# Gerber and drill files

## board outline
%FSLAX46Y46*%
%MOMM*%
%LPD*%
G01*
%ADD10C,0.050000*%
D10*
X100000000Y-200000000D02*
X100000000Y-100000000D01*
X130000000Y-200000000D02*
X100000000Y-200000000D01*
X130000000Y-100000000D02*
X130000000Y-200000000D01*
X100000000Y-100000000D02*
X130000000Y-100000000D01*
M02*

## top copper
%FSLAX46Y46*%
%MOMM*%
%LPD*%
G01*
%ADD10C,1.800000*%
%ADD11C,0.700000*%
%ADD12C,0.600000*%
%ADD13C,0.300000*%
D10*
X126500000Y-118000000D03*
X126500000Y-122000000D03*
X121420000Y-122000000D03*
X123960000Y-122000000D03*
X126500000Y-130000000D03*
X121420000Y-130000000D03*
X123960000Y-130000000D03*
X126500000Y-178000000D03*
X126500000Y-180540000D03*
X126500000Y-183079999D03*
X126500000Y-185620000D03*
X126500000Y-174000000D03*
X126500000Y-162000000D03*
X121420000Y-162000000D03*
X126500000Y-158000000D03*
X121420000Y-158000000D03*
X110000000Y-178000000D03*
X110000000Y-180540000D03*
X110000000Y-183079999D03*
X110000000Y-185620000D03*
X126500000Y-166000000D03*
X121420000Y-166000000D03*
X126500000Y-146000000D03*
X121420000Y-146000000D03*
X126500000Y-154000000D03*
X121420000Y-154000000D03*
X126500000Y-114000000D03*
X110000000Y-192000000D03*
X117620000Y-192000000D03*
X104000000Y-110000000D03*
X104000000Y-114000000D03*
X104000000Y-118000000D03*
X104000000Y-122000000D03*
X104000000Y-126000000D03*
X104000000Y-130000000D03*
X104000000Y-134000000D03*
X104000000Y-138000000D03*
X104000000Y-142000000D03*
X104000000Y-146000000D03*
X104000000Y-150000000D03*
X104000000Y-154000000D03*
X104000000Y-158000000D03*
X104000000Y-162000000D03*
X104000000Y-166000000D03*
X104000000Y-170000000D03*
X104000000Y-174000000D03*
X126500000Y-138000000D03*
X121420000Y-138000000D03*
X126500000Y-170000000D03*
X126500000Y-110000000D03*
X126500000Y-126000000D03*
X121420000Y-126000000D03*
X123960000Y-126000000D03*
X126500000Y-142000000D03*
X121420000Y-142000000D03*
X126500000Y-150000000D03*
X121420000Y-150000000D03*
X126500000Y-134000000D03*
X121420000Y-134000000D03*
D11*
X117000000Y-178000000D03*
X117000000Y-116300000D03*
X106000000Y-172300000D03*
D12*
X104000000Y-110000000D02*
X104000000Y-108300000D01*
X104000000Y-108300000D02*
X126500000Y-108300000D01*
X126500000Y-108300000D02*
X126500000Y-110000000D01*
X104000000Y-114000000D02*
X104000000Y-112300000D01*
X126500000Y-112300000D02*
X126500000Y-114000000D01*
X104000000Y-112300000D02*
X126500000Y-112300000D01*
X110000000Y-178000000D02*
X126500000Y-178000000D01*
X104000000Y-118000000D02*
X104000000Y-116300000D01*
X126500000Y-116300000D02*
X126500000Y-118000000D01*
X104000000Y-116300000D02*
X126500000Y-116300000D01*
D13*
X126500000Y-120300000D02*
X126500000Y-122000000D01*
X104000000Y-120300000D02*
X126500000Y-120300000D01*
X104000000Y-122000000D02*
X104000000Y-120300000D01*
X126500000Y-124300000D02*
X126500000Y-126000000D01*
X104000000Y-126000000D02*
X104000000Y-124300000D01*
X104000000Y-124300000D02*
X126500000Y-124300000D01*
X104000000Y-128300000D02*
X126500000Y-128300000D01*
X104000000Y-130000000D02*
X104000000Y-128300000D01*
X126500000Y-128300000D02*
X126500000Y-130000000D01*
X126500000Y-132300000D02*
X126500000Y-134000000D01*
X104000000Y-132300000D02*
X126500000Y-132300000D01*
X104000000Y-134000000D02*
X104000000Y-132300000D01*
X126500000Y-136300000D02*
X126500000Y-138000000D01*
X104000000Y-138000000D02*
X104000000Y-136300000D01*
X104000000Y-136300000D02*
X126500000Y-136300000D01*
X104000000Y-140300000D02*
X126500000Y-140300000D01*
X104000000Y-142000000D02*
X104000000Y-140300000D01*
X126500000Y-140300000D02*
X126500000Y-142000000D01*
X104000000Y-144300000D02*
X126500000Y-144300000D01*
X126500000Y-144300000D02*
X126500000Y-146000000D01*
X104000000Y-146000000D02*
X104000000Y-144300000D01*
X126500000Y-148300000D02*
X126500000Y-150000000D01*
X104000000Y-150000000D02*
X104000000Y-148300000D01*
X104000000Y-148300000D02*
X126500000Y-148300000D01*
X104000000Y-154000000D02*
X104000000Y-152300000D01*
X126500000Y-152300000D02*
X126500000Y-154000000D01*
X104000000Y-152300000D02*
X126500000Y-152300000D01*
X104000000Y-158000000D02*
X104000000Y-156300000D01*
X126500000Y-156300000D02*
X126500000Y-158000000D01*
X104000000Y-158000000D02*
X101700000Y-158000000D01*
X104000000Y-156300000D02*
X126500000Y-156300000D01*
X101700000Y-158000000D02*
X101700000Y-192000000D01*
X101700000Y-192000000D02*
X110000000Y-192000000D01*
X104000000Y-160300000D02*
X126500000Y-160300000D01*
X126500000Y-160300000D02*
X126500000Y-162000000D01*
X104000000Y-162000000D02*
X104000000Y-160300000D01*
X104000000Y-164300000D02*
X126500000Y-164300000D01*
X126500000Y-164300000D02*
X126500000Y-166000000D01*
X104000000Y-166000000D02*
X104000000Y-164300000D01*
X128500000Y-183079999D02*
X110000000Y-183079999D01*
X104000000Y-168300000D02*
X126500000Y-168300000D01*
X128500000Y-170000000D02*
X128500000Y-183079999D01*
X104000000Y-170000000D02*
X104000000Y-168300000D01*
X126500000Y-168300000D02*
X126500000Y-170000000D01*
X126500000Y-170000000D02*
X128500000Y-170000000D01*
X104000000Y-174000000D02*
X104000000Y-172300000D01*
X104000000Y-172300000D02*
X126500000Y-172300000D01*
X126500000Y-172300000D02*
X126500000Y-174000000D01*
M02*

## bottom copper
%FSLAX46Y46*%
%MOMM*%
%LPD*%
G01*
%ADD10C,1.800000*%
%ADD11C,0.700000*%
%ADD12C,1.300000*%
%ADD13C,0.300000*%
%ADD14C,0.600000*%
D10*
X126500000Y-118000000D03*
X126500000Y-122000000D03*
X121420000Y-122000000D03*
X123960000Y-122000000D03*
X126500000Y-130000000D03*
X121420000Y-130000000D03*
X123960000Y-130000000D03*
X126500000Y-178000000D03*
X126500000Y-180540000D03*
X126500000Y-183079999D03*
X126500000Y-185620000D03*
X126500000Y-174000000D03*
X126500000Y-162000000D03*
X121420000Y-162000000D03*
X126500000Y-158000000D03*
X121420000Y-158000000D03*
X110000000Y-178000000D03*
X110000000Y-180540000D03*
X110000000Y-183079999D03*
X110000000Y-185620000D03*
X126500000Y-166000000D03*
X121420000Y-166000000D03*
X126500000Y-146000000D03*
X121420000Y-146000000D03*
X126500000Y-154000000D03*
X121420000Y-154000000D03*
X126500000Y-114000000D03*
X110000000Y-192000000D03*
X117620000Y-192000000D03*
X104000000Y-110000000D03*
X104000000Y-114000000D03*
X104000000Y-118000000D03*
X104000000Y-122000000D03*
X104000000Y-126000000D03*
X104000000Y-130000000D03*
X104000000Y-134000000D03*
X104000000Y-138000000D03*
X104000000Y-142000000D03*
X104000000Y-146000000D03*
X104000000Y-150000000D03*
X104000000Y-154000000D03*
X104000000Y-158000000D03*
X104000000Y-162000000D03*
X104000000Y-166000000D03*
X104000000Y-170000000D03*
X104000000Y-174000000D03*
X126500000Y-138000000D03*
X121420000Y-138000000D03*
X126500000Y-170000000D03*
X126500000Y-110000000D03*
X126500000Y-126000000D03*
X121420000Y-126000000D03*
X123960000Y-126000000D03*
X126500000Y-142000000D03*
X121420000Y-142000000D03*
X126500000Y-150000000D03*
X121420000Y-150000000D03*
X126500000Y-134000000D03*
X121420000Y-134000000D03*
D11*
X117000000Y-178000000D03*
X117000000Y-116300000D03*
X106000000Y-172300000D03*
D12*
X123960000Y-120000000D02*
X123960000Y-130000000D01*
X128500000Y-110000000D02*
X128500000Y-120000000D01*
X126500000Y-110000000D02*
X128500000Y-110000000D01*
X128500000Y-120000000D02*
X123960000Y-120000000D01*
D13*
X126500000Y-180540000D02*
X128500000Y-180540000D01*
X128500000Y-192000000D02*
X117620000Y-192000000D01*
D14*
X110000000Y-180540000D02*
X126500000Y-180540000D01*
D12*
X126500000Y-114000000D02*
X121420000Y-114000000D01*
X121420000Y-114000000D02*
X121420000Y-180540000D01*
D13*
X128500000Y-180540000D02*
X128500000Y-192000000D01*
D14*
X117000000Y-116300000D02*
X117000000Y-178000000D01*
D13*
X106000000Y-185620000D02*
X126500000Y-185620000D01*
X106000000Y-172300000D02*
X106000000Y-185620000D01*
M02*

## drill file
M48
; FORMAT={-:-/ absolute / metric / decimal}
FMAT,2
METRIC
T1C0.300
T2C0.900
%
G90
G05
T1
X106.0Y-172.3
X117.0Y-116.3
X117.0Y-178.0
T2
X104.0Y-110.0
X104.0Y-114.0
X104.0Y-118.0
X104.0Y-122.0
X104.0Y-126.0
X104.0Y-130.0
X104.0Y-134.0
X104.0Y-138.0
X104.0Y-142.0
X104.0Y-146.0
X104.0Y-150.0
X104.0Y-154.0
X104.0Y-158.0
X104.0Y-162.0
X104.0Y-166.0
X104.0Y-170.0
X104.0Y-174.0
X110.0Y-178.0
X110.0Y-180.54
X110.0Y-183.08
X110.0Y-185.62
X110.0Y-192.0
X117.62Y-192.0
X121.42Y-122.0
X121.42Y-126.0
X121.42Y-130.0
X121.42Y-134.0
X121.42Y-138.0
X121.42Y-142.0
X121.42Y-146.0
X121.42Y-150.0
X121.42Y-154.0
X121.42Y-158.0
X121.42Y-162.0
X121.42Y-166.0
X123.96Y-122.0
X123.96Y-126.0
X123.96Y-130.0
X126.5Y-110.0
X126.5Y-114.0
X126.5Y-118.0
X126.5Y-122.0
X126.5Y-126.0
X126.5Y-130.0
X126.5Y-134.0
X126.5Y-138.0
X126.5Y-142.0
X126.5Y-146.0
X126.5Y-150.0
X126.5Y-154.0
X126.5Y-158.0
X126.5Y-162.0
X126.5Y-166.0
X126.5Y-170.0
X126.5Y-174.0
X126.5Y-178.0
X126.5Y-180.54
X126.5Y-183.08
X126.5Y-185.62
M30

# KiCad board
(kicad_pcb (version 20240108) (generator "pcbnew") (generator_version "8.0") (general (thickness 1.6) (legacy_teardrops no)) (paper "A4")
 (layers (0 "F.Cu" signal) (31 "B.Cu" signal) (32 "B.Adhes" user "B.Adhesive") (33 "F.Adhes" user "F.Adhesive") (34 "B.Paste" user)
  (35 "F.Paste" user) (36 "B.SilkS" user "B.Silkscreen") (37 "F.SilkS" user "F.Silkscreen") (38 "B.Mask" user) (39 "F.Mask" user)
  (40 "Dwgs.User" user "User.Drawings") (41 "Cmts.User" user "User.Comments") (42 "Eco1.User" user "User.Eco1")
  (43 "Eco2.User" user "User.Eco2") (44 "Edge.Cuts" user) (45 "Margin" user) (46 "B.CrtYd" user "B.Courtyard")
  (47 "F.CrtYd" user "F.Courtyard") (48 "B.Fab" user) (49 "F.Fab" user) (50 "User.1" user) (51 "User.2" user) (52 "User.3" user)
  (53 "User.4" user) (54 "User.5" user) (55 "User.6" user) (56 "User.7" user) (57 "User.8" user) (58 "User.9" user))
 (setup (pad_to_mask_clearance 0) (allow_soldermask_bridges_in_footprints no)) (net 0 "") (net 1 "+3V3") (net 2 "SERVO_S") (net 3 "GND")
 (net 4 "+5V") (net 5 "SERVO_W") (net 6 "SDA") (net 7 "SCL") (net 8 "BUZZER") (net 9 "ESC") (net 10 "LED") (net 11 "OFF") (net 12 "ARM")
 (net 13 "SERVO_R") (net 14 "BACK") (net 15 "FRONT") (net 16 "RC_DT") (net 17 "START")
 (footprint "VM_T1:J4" (layer "F.Cu") (at 100 100)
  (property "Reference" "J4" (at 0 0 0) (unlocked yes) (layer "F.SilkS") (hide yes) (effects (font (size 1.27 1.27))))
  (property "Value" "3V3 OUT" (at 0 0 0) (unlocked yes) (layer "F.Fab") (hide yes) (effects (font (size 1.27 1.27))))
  (pad "1" thru_hole circle (at 26.5 18) (size 1.8 1.8) (drill 0.9) (layers "*.Cu" "*.Mask") (remove_unused_layers no) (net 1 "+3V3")))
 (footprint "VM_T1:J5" (layer "F.Cu") (at 100 100)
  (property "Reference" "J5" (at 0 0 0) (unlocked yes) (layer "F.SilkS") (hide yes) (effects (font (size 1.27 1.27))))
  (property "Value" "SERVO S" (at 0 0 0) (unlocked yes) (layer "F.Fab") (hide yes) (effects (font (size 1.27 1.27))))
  (pad "1" thru_hole circle (at 26.5 22) (size 1.8 1.8) (drill 0.9) (layers "*.Cu" "*.Mask") (remove_unused_layers no) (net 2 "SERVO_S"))
  (pad "2" thru_hole circle (at 21.42 22) (size 1.8 1.8) (drill 0.9) (layers "*.Cu" "*.Mask") (remove_unused_layers no) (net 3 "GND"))
  (pad "3" thru_hole circle (at 23.96 22) (size 1.8 1.8) (drill 0.9) (layers "*.Cu" "*.Mask") (remove_unused_layers no) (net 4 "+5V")))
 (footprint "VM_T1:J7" (layer "F.Cu") (at 100 100)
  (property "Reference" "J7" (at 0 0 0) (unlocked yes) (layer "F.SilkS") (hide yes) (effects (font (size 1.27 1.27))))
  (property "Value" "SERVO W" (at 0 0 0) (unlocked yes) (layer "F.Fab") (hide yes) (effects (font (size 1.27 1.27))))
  (pad "1" thru_hole circle (at 26.5 30) (size 1.8 1.8) (drill 0.9) (layers "*.Cu" "*.Mask") (remove_unused_layers no) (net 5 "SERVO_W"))
  (pad "2" thru_hole circle (at 21.42 30) (size 1.8 1.8) (drill 0.9) (layers "*.Cu" "*.Mask") (remove_unused_layers no) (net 3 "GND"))
  (pad "3" thru_hole circle (at 23.96 30) (size 1.8 1.8) (drill 0.9) (layers "*.Cu" "*.Mask") (remove_unused_layers no) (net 4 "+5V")))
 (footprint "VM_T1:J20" (layer "F.Cu") (at 100 100)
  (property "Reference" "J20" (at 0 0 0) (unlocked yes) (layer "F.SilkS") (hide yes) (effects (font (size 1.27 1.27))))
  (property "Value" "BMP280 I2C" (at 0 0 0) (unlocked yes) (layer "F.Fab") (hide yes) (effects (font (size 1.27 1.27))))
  (pad "1" thru_hole circle (at 26.5 78) (size 1.8 1.8) (drill 0.9) (layers "*.Cu" "*.Mask") (remove_unused_layers no) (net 1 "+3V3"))
  (pad "2" thru_hole circle (at 26.5 80.54) (size 1.8 1.8) (drill 0.9) (layers "*.Cu" "*.Mask") (remove_unused_layers no) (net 3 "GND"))
  (pad "3" thru_hole circle (at 26.5 83.079999) (size 1.8 1.8) (drill 0.9) (layers "*.Cu" "*.Mask") (remove_unused_layers no) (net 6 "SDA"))
  (pad "4" thru_hole circle (at 26.5 85.62) (size 1.8 1.8) (drill 0.9) (layers "*.Cu" "*.Mask") (remove_unused_layers no) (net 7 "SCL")))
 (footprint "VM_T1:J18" (layer "F.Cu") (at 100 100)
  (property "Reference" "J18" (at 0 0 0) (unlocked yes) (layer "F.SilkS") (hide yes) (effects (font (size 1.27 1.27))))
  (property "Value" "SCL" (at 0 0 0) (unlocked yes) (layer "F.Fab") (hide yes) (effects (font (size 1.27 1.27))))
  (pad "1" thru_hole circle (at 26.5 74) (size 1.8 1.8) (drill 0.9) (layers "*.Cu" "*.Mask") (remove_unused_layers no) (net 7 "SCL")))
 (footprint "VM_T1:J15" (layer "F.Cu") (at 100 100)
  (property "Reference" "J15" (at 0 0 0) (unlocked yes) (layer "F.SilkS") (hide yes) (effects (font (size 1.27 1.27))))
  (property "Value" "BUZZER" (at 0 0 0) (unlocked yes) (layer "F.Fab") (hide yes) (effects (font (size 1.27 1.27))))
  (pad "1" thru_hole circle (at 26.5 62) (size 1.8 1.8) (drill 0.9) (layers "*.Cu" "*.Mask") (remove_unused_layers no) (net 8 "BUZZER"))
  (pad "2" thru_hole circle (at 21.42 62) (size 1.8 1.8) (drill 0.9) (layers "*.Cu" "*.Mask") (remove_unused_layers no) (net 3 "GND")))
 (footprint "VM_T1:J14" (layer "F.Cu") (at 100 100)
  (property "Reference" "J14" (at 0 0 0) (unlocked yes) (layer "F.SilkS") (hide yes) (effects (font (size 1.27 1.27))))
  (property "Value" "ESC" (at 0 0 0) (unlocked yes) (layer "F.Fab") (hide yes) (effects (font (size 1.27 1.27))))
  (pad "1" thru_hole circle (at 26.5 58) (size 1.8 1.8) (drill 0.9) (layers "*.Cu" "*.Mask") (remove_unused_layers no) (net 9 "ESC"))
  (pad "2" thru_hole circle (at 21.42 58) (size 1.8 1.8) (drill 0.9) (layers "*.Cu" "*.Mask") (remove_unused_layers no) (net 3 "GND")))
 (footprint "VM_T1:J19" (layer "F.Cu") (at 100 100)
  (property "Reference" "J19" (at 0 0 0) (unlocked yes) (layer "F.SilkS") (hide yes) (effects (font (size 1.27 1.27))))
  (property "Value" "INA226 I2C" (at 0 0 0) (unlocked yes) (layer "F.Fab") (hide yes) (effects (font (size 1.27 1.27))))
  (pad "1" thru_hole circle (at 10 78) (size 1.8 1.8) (drill 0.9) (layers "*.Cu" "*.Mask") (remove_unused_layers no) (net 1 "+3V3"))
  (pad "2" thru_hole circle (at 10 80.54) (size 1.8 1.8) (drill 0.9) (layers "*.Cu" "*.Mask") (remove_unused_layers no) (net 3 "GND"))
  (pad "3" thru_hole circle (at 10 83.079999) (size 1.8 1.8) (drill 0.9) (layers "*.Cu" "*.Mask") (remove_unused_layers no) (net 6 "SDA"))
  (pad "4" thru_hole circle (at 10 85.62) (size 1.8 1.8) (drill 0.9) (layers "*.Cu" "*.Mask") (remove_unused_layers no) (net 7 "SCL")))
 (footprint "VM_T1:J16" (layer "F.Cu") (at 100 100)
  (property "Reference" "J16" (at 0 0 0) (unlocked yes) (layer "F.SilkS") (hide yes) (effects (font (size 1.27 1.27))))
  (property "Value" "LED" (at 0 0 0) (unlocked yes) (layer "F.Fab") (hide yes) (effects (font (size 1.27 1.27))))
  (pad "1" thru_hole circle (at 26.5 66) (size 1.8 1.8) (drill 0.9) (layers "*.Cu" "*.Mask") (remove_unused_layers no) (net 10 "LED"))
  (pad "2" thru_hole circle (at 21.42 66) (size 1.8 1.8) (drill 0.9) (layers "*.Cu" "*.Mask") (remove_unused_layers no) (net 3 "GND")))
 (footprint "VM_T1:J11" (layer "F.Cu") (at 100 100)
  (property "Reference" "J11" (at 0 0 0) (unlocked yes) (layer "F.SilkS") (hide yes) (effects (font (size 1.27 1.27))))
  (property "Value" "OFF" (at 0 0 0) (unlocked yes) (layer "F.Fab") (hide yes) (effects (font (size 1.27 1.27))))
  (pad "1" thru_hole circle (at 26.5 46) (size 1.8 1.8) (drill 0.9) (layers "*.Cu" "*.Mask") (remove_unused_layers no) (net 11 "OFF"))
  (pad "2" thru_hole circle (at 21.42 46) (size 1.8 1.8) (drill 0.9) (layers "*.Cu" "*.Mask") (remove_unused_layers no) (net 3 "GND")))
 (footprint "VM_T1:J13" (layer "F.Cu") (at 100 100)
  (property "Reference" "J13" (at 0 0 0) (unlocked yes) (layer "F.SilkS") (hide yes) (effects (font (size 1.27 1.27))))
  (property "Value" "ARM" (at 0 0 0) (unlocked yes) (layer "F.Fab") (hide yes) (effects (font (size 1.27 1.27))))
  (pad "1" thru_hole circle (at 26.5 54) (size 1.8 1.8) (drill 0.9) (layers "*.Cu" "*.Mask") (remove_unused_layers no) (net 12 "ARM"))
  (pad "2" thru_hole circle (at 21.42 54) (size 1.8 1.8) (drill 0.9) (layers "*.Cu" "*.Mask") (remove_unused_layers no) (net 3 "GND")))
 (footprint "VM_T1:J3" (layer "F.Cu") (at 100 100)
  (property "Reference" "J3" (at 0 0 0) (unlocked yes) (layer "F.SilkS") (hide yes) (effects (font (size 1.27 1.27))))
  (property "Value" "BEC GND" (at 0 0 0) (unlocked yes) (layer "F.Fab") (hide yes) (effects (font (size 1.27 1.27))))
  (pad "1" thru_hole circle (at 26.5 14) (size 1.8 1.8) (drill 0.9) (layers "*.Cu" "*.Mask") (remove_unused_layers no) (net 3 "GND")))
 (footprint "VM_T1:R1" (layer "F.Cu") (at 100 100)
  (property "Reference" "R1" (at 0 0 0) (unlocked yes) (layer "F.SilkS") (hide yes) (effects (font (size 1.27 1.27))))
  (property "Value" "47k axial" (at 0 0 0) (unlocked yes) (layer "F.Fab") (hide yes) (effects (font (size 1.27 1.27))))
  (pad "1" thru_hole circle (at 10 92) (size 1.8 1.8) (drill 0.9) (layers "*.Cu" "*.Mask") (remove_unused_layers no) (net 9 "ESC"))
  (pad "2" thru_hole circle (at 17.62 92) (size 1.8 1.8) (drill 0.9) (layers "*.Cu" "*.Mask") (remove_unused_layers no) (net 3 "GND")))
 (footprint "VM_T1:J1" (layer "F.Cu") (at 100 100)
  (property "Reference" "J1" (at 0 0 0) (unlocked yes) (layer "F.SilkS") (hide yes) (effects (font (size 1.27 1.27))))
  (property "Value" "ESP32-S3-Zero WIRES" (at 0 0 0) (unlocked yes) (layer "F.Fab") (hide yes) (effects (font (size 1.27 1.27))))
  (pad "1" thru_hole circle (at 4 10) (size 1.8 1.8) (drill 0.9) (layers "*.Cu" "*.Mask") (remove_unused_layers no) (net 4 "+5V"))
  (pad "2" thru_hole circle (at 4 14) (size 1.8 1.8) (drill 0.9) (layers "*.Cu" "*.Mask") (remove_unused_layers no) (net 3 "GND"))
  (pad "3" thru_hole circle (at 4 18) (size 1.8 1.8) (drill 0.9) (layers "*.Cu" "*.Mask") (remove_unused_layers no) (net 1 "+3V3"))
  (pad "4" thru_hole circle (at 4 22) (size 1.8 1.8) (drill 0.9) (layers "*.Cu" "*.Mask") (remove_unused_layers no) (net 2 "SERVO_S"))
  (pad "5" thru_hole circle (at 4 26) (size 1.8 1.8) (drill 0.9) (layers "*.Cu" "*.Mask") (remove_unused_layers no) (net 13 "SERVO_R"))
  (pad "6" thru_hole circle (at 4 30) (size 1.8 1.8) (drill 0.9) (layers "*.Cu" "*.Mask") (remove_unused_layers no) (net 5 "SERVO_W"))
  (pad "7" thru_hole circle (at 4 34) (size 1.8 1.8) (drill 0.9) (layers "*.Cu" "*.Mask") (remove_unused_layers no) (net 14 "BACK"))
  (pad "8" thru_hole circle (at 4 38) (size 1.8 1.8) (drill 0.9) (layers "*.Cu" "*.Mask") (remove_unused_layers no) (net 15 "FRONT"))
  (pad "9" thru_hole circle (at 4 42) (size 1.8 1.8) (drill 0.9) (layers "*.Cu" "*.Mask") (remove_unused_layers no) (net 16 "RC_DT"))
  (pad "10" thru_hole circle (at 4 46) (size 1.8 1.8) (drill 0.9) (layers "*.Cu" "*.Mask") (remove_unused_layers no) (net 11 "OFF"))
  (pad "11" thru_hole circle (at 4 50) (size 1.8 1.8) (drill 0.9) (layers "*.Cu" "*.Mask") (remove_unused_layers no) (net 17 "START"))
  (pad "12" thru_hole circle (at 4 54) (size 1.8 1.8) (drill 0.9) (layers "*.Cu" "*.Mask") (remove_unused_layers no) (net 12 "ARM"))
  (pad "13" thru_hole circle (at 4 58) (size 1.8 1.8) (drill 0.9) (layers "*.Cu" "*.Mask") (remove_unused_layers no) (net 9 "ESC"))
  (pad "14" thru_hole circle (at 4 62) (size 1.8 1.8) (drill 0.9) (layers "*.Cu" "*.Mask") (remove_unused_layers no) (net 8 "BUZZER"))
  (pad "15" thru_hole circle (at 4 66) (size 1.8 1.8) (drill 0.9) (layers "*.Cu" "*.Mask") (remove_unused_layers no) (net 10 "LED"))
  (pad "16" thru_hole circle (at 4 70) (size 1.8 1.8) (drill 0.9) (layers "*.Cu" "*.Mask") (remove_unused_layers no) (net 6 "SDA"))
  (pad "17" thru_hole circle (at 4 74) (size 1.8 1.8) (drill 0.9) (layers "*.Cu" "*.Mask") (remove_unused_layers no) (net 7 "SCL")))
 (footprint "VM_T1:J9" (layer "F.Cu") (at 100 100)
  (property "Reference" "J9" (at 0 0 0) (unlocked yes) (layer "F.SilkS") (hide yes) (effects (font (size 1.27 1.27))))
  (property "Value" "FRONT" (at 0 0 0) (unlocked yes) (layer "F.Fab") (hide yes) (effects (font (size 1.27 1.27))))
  (pad "1" thru_hole circle (at 26.5 38) (size 1.8 1.8) (drill 0.9) (layers "*.Cu" "*.Mask") (remove_unused_layers no) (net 15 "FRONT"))
  (pad "2" thru_hole circle (at 21.42 38) (size 1.8 1.8) (drill 0.9) (layers "*.Cu" "*.Mask") (remove_unused_layers no) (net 3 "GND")))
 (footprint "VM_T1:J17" (layer "F.Cu") (at 100 100)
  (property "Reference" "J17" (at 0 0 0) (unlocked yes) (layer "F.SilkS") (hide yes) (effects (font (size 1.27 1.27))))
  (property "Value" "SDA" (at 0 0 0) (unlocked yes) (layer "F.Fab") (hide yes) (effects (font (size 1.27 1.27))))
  (pad "1" thru_hole circle (at 26.5 70) (size 1.8 1.8) (drill 0.9) (layers "*.Cu" "*.Mask") (remove_unused_layers no) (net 6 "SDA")))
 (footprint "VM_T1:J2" (layer "F.Cu") (at 100 100)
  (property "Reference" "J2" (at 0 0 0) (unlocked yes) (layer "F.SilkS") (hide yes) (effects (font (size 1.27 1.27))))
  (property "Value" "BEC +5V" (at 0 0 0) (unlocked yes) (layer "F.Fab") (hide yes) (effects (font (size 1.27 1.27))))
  (pad "1" thru_hole circle (at 26.5 10) (size 1.8 1.8) (drill 0.9) (layers "*.Cu" "*.Mask") (remove_unused_layers no) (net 4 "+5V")))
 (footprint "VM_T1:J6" (layer "F.Cu") (at 100 100)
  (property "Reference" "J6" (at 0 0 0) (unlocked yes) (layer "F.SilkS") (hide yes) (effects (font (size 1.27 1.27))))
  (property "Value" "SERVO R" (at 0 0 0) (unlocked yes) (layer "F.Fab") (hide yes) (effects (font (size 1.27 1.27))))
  (pad "1" thru_hole circle (at 26.5 26) (size 1.8 1.8) (drill 0.9) (layers "*.Cu" "*.Mask") (remove_unused_layers no) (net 13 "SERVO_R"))
  (pad "2" thru_hole circle (at 21.42 26) (size 1.8 1.8) (drill 0.9) (layers "*.Cu" "*.Mask") (remove_unused_layers no) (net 3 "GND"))
  (pad "3" thru_hole circle (at 23.96 26) (size 1.8 1.8) (drill 0.9) (layers "*.Cu" "*.Mask") (remove_unused_layers no) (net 4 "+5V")))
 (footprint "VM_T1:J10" (layer "F.Cu") (at 100 100)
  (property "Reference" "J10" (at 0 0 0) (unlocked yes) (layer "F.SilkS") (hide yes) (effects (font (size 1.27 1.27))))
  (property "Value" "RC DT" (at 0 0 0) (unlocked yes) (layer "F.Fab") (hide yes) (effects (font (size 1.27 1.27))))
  (pad "1" thru_hole circle (at 26.5 42) (size 1.8 1.8) (drill 0.9) (layers "*.Cu" "*.Mask") (remove_unused_layers no) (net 16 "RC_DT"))
  (pad "2" thru_hole circle (at 21.42 42) (size 1.8 1.8) (drill 0.9) (layers "*.Cu" "*.Mask") (remove_unused_layers no) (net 3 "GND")))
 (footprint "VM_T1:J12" (layer "F.Cu") (at 100 100)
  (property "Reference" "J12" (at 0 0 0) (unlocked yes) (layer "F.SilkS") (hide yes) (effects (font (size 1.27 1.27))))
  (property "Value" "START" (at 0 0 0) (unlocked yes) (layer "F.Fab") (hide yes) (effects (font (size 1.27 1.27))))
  (pad "1" thru_hole circle (at 26.5 50) (size 1.8 1.8) (drill 0.9) (layers "*.Cu" "*.Mask") (remove_unused_layers no) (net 17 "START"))
  (pad "2" thru_hole circle (at 21.42 50) (size 1.8 1.8) (drill 0.9) (layers "*.Cu" "*.Mask") (remove_unused_layers no) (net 3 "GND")))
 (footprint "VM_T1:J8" (layer "F.Cu") (at 100 100)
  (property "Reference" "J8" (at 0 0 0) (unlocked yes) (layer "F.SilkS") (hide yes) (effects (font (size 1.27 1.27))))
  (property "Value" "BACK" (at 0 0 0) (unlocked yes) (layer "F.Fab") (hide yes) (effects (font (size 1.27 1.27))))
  (pad "1" thru_hole circle (at 26.5 34) (size 1.8 1.8) (drill 0.9) (layers "*.Cu" "*.Mask") (remove_unused_layers no) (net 14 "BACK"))
  (pad "2" thru_hole circle (at 21.42 34) (size 1.8 1.8) (drill 0.9) (layers "*.Cu" "*.Mask") (remove_unused_layers no) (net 3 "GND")))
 (gr_line (start 100 200) (end 100 100) (stroke (width 0.05) (type default)) (layer "Edge.Cuts"))
 (gr_line (start 130 200) (end 100 200) (stroke (width 0.05) (type default)) (layer "Edge.Cuts"))
 (gr_line (start 130 100) (end 130 200) (stroke (width 0.05) (type default)) (layer "Edge.Cuts"))
 (gr_line (start 100 100) (end 130 100) (stroke (width 0.05) (type default)) (layer "Edge.Cuts"))
 (segment (start 104 110) (end 104 108.3) (width 0.6) (layer "F.Cu") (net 4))
 (segment (start 104 108.3) (end 126.5 108.3) (width 0.6) (layer "F.Cu") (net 4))
 (segment (start 126.5 108.3) (end 126.5 110) (width 0.6) (layer "F.Cu") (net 4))
 (segment (start 123.96 120) (end 123.96 130) (width 1.3) (layer "B.Cu") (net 4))
 (segment (start 128.5 110) (end 128.5 120) (width 1.3) (layer "B.Cu") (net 4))
 (segment (start 126.5 110) (end 128.5 110) (width 1.3) (layer "B.Cu") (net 4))
 (segment (start 128.5 120) (end 123.96 120) (width 1.3) (layer "B.Cu") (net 4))
 (segment (start 104 114) (end 104 112.3) (width 0.6) (layer "F.Cu") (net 3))
 (segment (start 126.5 112.3) (end 126.5 114) (width 0.6) (layer "F.Cu") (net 3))
 (segment (start 104 112.3) (end 126.5 112.3) (width 0.6) (layer "F.Cu") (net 3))
 (segment (start 126.5 180.54) (end 128.5 180.54) (width 0.3) (layer "B.Cu") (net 3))
 (segment (start 128.5 192) (end 117.62 192) (width 0.3) (layer "B.Cu") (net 3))
 (segment (start 110 180.54) (end 126.5 180.54) (width 0.6) (layer "B.Cu") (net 3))
 (segment (start 126.5 114) (end 121.42 114) (width 1.3) (layer "B.Cu") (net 3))
 (segment (start 121.42 114) (end 121.42 180.54) (width 1.3) (layer "B.Cu") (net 3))
 (segment (start 128.5 180.54) (end 128.5 192) (width 0.3) (layer "B.Cu") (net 3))
 (segment (start 110 178) (end 126.5 178) (width 0.6) (layer "F.Cu") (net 1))
 (segment (start 104 118) (end 104 116.3) (width 0.6) (layer "F.Cu") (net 1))
 (segment (start 126.5 116.3) (end 126.5 118) (width 0.6) (layer "F.Cu") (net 1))
 (segment (start 104 116.3) (end 126.5 116.3) (width 0.6) (layer "F.Cu") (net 1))
 (via (at 117 178) (size 0.7) (drill 0.3) (layers "F.Cu" "B.Cu") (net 1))
 (via (at 117 116.3) (size 0.7) (drill 0.3) (layers "F.Cu" "B.Cu") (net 1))
 (segment (start 117 116.3) (end 117 178) (width 0.6) (layer "B.Cu") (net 1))
 (segment (start 126.5 120.3) (end 126.5 122) (width 0.3) (layer "F.Cu") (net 2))
 (segment (start 104 120.3) (end 126.5 120.3) (width 0.3) (layer "F.Cu") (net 2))
 (segment (start 104 122) (end 104 120.3) (width 0.3) (layer "F.Cu") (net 2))
 (segment (start 126.5 124.3) (end 126.5 126) (width 0.3) (layer "F.Cu") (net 13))
 (segment (start 104 126) (end 104 124.3) (width 0.3) (layer "F.Cu") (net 13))
 (segment (start 104 124.3) (end 126.5 124.3) (width 0.3) (layer "F.Cu") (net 13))
 (segment (start 104 128.3) (end 126.5 128.3) (width 0.3) (layer "F.Cu") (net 5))
 (segment (start 104 130) (end 104 128.3) (width 0.3) (layer "F.Cu") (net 5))
 (segment (start 126.5 128.3) (end 126.5 130) (width 0.3) (layer "F.Cu") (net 5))
 (segment (start 126.5 132.3) (end 126.5 134) (width 0.3) (layer "F.Cu") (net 14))
 (segment (start 104 132.3) (end 126.5 132.3) (width 0.3) (layer "F.Cu") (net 14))
 (segment (start 104 134) (end 104 132.3) (width 0.3) (layer "F.Cu") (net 14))
 (segment (start 126.5 136.3) (end 126.5 138) (width 0.3) (layer "F.Cu") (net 15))
 (segment (start 104 138) (end 104 136.3) (width 0.3) (layer "F.Cu") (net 15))
 (segment (start 104 136.3) (end 126.5 136.3) (width 0.3) (layer "F.Cu") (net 15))
 (segment (start 104 140.3) (end 126.5 140.3) (width 0.3) (layer "F.Cu") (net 16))
 (segment (start 104 142) (end 104 140.3) (width 0.3) (layer "F.Cu") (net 16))
 (segment (start 126.5 140.3) (end 126.5 142) (width 0.3) (layer "F.Cu") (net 16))
 (segment (start 104 144.3) (end 126.5 144.3) (width 0.3) (layer "F.Cu") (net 11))
 (segment (start 126.5 144.3) (end 126.5 146) (width 0.3) (layer "F.Cu") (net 11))
 (segment (start 104 146) (end 104 144.3) (width 0.3) (layer "F.Cu") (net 11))
 (segment (start 126.5 148.3) (end 126.5 150) (width 0.3) (layer "F.Cu") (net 17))
 (segment (start 104 150) (end 104 148.3) (width 0.3) (layer "F.Cu") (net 17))
 (segment (start 104 148.3) (end 126.5 148.3) (width 0.3) (layer "F.Cu") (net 17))
 (segment (start 104 154) (end 104 152.3) (width 0.3) (layer "F.Cu") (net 12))
 (segment (start 126.5 152.3) (end 126.5 154) (width 0.3) (layer "F.Cu") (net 12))
 (segment (start 104 152.3) (end 126.5 152.3) (width 0.3) (layer "F.Cu") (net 12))
 (segment (start 104 158) (end 104 156.3) (width 0.3) (layer "F.Cu") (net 9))
 (segment (start 126.5 156.3) (end 126.5 158) (width 0.3) (layer "F.Cu") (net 9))
 (segment (start 104 158) (end 101.7 158) (width 0.3) (layer "F.Cu") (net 9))
 (segment (start 104 156.3) (end 126.5 156.3) (width 0.3) (layer "F.Cu") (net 9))
 (segment (start 101.7 158) (end 101.7 192) (width 0.3) (layer "F.Cu") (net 9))
 (segment (start 101.7 192) (end 110 192) (width 0.3) (layer "F.Cu") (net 9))
 (segment (start 104 160.3) (end 126.5 160.3) (width 0.3) (layer "F.Cu") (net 8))
 (segment (start 126.5 160.3) (end 126.5 162) (width 0.3) (layer "F.Cu") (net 8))
 (segment (start 104 162) (end 104 160.3) (width 0.3) (layer "F.Cu") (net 8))
 (segment (start 104 164.3) (end 126.5 164.3) (width 0.3) (layer "F.Cu") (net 10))
 (segment (start 126.5 164.3) (end 126.5 166) (width 0.3) (layer "F.Cu") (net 10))
 (segment (start 104 166) (end 104 164.3) (width 0.3) (layer "F.Cu") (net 10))
 (segment (start 128.5 183.079999) (end 110 183.079999) (width 0.3) (layer "F.Cu") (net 6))
 (segment (start 104 168.3) (end 126.5 168.3) (width 0.3) (layer "F.Cu") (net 6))
 (segment (start 128.5 170) (end 128.5 183.079999) (width 0.3) (layer "F.Cu") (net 6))
 (segment (start 104 170) (end 104 168.3) (width 0.3) (layer "F.Cu") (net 6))
 (segment (start 126.5 168.3) (end 126.5 170) (width 0.3) (layer "F.Cu") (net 6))
 (segment (start 126.5 170) (end 128.5 170) (width 0.3) (layer "F.Cu") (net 6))
 (segment (start 104 174) (end 104 172.3) (width 0.3) (layer "F.Cu") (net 7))
 (segment (start 104 172.3) (end 126.5 172.3) (width 0.3) (layer "F.Cu") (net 7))
 (segment (start 126.5 172.3) (end 126.5 174) (width 0.3) (layer "F.Cu") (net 7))
 (via (at 106 172.3) (size 0.7) (drill 0.3) (layers "F.Cu" "B.Cu") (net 7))
 (segment (start 106 185.62) (end 126.5 185.62) (width 0.3) (layer "B.Cu") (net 7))
 (segment (start 106 172.3) (end 106 185.62) (width 0.3) (layer "B.Cu") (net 7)))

